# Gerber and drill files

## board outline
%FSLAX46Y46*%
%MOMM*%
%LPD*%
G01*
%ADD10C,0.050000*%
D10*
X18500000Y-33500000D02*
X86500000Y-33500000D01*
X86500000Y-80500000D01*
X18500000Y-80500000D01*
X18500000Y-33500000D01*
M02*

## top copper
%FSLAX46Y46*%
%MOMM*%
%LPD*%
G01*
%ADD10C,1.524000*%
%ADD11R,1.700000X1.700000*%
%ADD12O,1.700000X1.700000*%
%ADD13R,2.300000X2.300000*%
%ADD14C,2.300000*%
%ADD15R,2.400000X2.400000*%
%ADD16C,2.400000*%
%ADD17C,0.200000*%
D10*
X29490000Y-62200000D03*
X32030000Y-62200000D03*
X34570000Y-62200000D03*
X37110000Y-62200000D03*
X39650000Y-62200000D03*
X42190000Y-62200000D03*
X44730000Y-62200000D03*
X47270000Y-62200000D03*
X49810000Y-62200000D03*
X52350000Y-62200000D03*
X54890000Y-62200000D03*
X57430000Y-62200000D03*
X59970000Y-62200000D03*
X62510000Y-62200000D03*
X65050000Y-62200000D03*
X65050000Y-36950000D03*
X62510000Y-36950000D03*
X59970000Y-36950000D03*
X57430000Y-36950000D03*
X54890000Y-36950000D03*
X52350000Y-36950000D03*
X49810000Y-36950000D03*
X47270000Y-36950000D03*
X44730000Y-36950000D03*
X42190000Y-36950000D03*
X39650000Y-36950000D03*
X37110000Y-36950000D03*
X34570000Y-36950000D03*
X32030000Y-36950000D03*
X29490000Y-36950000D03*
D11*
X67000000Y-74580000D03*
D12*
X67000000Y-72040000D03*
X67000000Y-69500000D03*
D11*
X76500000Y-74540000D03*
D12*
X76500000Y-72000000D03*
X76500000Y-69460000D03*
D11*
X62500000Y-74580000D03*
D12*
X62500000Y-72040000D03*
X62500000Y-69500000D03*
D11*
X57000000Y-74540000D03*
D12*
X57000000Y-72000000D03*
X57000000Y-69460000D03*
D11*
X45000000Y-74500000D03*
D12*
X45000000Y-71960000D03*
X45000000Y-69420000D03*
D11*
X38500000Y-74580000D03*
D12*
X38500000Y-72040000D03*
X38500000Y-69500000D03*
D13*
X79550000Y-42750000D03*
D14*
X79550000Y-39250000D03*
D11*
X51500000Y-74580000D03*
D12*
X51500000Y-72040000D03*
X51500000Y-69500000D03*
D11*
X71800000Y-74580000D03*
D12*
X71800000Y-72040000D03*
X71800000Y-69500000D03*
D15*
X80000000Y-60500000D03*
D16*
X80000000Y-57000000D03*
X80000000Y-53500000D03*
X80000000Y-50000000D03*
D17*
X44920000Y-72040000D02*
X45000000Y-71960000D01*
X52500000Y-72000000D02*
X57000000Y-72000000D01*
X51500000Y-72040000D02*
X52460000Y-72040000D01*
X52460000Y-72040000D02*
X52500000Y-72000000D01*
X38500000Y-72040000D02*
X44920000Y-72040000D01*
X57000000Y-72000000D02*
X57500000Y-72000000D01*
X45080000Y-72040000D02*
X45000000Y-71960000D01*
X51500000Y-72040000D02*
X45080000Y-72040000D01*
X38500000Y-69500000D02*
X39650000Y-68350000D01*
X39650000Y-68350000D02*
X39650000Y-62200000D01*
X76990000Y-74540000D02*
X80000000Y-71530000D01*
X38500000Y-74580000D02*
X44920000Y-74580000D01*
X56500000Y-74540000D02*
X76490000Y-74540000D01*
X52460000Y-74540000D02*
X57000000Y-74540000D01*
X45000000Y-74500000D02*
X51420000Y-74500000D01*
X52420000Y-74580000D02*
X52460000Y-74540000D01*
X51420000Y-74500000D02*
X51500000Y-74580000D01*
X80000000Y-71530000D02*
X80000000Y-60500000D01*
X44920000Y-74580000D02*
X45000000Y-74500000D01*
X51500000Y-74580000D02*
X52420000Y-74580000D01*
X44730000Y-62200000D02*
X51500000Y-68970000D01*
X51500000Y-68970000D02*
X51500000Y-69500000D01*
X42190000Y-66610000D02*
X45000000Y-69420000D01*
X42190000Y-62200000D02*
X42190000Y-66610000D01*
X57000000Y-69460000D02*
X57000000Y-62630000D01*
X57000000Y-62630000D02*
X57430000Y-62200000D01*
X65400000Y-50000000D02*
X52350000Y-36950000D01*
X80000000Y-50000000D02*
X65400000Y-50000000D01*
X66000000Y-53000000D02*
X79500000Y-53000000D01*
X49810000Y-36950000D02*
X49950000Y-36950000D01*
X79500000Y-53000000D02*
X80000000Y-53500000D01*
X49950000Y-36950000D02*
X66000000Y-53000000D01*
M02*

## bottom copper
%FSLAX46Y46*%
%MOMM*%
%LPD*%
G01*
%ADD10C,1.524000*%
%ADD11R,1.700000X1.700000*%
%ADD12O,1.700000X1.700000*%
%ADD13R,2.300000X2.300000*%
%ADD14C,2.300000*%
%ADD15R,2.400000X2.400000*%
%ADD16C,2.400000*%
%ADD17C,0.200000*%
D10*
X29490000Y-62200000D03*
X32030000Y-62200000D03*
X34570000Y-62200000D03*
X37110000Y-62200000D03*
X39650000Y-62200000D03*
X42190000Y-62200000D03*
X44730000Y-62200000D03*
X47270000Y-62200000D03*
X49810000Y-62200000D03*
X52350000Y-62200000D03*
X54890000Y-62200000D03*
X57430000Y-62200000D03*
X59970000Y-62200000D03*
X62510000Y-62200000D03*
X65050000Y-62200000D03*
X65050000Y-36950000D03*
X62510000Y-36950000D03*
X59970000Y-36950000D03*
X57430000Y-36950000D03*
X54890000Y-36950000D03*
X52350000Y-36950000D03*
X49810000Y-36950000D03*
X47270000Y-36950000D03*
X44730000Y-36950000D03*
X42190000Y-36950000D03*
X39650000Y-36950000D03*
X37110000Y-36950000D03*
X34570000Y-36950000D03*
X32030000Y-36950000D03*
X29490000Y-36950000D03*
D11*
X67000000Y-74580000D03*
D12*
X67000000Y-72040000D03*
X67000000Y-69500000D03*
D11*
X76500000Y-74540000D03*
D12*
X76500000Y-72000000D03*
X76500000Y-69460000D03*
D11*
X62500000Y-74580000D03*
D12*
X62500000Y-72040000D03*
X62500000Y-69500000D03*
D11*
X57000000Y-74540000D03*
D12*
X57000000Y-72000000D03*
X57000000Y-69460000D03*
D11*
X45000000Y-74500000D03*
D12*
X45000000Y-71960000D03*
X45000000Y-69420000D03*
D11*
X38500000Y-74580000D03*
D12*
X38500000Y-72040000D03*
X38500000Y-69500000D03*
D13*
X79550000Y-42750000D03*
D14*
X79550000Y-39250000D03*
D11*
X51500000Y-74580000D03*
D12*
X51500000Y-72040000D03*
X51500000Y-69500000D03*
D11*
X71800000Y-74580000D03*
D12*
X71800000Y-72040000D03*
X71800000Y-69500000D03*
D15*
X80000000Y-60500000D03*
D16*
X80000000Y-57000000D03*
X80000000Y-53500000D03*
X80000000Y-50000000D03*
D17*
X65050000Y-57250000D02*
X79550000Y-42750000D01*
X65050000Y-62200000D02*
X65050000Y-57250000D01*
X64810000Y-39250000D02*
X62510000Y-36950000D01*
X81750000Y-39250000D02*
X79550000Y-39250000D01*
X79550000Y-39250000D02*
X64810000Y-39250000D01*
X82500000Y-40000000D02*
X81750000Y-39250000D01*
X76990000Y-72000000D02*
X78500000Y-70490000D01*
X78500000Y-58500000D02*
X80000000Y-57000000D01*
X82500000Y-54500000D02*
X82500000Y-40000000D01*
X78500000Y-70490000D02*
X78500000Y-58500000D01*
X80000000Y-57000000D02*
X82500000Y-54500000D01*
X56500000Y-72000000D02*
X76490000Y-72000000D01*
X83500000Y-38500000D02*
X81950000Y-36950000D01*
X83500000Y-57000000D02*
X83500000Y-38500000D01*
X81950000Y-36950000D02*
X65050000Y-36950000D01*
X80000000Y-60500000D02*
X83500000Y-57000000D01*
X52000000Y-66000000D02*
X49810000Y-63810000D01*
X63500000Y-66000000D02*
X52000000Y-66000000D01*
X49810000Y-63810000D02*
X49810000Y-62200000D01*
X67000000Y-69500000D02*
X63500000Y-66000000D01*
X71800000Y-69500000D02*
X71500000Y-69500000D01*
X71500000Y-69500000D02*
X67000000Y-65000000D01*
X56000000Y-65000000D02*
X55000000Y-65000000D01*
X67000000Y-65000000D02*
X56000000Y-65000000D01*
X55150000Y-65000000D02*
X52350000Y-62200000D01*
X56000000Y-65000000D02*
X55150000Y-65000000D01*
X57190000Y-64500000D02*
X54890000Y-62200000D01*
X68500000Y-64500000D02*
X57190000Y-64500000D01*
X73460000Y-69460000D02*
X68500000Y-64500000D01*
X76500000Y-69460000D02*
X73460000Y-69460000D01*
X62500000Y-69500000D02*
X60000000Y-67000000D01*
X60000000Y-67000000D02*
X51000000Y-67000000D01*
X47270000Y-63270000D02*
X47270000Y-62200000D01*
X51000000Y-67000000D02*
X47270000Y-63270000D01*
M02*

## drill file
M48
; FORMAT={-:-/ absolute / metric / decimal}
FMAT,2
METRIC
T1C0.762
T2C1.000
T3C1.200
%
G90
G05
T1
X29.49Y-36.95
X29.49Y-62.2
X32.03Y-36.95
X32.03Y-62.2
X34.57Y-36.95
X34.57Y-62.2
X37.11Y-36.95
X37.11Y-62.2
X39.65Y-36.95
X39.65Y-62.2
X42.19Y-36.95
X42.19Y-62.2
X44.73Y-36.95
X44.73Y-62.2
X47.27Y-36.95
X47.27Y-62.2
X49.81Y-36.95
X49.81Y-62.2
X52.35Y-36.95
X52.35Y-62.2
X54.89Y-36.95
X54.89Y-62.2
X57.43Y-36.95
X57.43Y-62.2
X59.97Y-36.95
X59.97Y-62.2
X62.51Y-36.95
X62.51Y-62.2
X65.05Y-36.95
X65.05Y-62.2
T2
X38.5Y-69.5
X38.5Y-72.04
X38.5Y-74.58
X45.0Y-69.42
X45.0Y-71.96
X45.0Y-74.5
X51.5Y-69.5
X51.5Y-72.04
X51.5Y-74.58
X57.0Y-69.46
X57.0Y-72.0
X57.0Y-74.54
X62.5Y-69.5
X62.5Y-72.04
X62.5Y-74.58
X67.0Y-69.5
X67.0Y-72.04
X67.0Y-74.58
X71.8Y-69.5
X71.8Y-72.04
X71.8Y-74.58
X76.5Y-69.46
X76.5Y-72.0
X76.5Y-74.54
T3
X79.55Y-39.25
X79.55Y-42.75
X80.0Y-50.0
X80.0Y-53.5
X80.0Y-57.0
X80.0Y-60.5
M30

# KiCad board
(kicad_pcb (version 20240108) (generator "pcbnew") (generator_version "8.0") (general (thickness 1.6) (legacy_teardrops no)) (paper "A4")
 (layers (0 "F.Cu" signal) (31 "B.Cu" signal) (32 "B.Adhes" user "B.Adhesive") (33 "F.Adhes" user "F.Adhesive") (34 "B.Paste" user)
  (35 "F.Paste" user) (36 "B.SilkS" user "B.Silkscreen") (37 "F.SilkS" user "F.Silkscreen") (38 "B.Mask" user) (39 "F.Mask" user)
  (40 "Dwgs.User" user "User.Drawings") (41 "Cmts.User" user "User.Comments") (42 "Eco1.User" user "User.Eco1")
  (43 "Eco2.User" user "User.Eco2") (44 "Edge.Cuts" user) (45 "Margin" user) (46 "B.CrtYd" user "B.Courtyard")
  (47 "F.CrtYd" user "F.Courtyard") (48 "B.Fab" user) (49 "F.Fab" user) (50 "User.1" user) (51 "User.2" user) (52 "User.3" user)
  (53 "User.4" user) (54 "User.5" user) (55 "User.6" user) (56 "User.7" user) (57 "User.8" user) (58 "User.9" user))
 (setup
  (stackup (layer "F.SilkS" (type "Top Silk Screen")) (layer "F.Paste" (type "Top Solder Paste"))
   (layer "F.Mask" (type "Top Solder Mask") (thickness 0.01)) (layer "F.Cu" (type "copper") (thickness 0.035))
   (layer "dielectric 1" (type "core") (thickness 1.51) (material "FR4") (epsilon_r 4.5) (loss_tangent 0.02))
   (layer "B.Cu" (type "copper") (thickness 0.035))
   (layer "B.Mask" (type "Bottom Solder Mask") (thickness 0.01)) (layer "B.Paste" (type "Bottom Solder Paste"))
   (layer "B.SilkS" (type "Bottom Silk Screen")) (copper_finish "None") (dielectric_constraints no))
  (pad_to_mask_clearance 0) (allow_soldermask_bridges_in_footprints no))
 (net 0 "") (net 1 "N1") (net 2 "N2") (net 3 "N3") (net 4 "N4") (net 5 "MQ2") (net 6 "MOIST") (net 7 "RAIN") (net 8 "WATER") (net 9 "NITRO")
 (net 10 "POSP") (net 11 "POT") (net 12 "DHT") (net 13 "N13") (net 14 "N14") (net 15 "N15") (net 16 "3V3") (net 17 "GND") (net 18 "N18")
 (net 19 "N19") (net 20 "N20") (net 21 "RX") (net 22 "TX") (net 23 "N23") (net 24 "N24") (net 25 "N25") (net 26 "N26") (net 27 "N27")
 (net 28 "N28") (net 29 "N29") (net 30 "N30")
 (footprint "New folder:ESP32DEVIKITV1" (layer "F.Cu") (at 29.49 62.2)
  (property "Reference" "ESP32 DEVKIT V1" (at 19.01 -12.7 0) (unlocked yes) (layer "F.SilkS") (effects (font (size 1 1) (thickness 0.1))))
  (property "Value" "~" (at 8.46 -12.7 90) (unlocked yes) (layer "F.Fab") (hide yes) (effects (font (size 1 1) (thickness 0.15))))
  (pad "1" thru_hole circle (at 0 0) (size 1.524 1.524) (drill 0.762) (layers "*.Cu" "*.Mask") (remove_unused_layers no) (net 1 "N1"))
  (pad "2" thru_hole circle (at 2.54 0) (size 1.524 1.524) (drill 0.762) (layers "*.Cu" "*.Mask") (remove_unused_layers no) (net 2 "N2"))
  (pad "3" thru_hole circle (at 5.08 0) (size 1.524 1.524) (drill 0.762) (layers "*.Cu" "*.Mask") (remove_unused_layers no) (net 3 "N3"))
  (pad "4" thru_hole circle (at 7.62 0) (size 1.524 1.524) (drill 0.762) (layers "*.Cu" "*.Mask") (remove_unused_layers no) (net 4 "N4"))
  (pad "5" thru_hole circle (at 10.16 0) (size 1.524 1.524) (drill 0.762) (layers "*.Cu" "*.Mask") (remove_unused_layers no) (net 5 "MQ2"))
  (pad "6" thru_hole circle (at 12.7 0) (size 1.524 1.524) (drill 0.762) (layers "*.Cu" "*.Mask") (remove_unused_layers no) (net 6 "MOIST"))
  (pad "7" thru_hole circle (at 15.24 0) (size 1.524 1.524) (drill 0.762) (layers "*.Cu" "*.Mask") (remove_unused_layers no) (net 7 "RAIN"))
  (pad "8" thru_hole circle (at 17.78 0) (size 1.524 1.524) (drill 0.762) (layers "*.Cu" "*.Mask") (remove_unused_layers no) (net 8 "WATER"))
  (pad "9" thru_hole circle (at 20.32 0) (size 1.524 1.524) (drill 0.762) (layers "*.Cu" "*.Mask") (remove_unused_layers no) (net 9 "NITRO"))
  (pad "10" thru_hole circle (at 22.86 0) (size 1.524 1.524) (drill 0.762) (layers "*.Cu" "*.Mask") (remove_unused_layers no)
   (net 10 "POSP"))
  (pad "11" thru_hole circle (at 25.4 0) (size 1.524 1.524) (drill 0.762) (layers "*.Cu" "*.Mask") (remove_unused_layers no) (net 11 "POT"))
  (pad "12" thru_hole circle (at 27.94 0) (size 1.524 1.524) (drill 0.762) (layers "*.Cu" "*.Mask") (remove_unused_layers no) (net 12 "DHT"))
  (pad "13" thru_hole circle (at 30.48 0) (size 1.524 1.524) (drill 0.762) (layers "*.Cu" "*.Mask") (remove_unused_layers no) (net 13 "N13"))
  (pad "14" thru_hole circle (at 33.02 0) (size 1.524 1.524) (drill 0.762) (layers "*.Cu" "*.Mask") (remove_unused_layers no) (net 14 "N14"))
  (pad "15" thru_hole circle (at 35.56 0) (size 1.524 1.524) (drill 0.762) (layers "*.Cu" "*.Mask") (remove_unused_layers no) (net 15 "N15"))
  (pad "16" thru_hole circle (at 35.56 -25.25) (size 1.524 1.524) (drill 0.762) (layers "*.Cu" "*.Mask") (remove_unused_layers no)
   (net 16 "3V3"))
  (pad "17" thru_hole circle (at 33.02 -25.25) (size 1.524 1.524) (drill 0.762) (layers "*.Cu" "*.Mask") (remove_unused_layers no)
   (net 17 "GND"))
  (pad "18" thru_hole circle (at 30.48 -25.25) (size 1.524 1.524) (drill 0.762) (layers "*.Cu" "*.Mask") (remove_unused_layers no)
   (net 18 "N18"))
  (pad "19" thru_hole circle (at 27.94 -25.25) (size 1.524 1.524) (drill 0.762) (layers "*.Cu" "*.Mask") (remove_unused_layers no)
   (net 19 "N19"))
  (pad "20" thru_hole circle (at 25.4 -25.25) (size 1.524 1.524) (drill 0.762) (layers "*.Cu" "*.Mask") (remove_unused_layers no)
   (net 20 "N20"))
  (pad "21" thru_hole circle (at 22.86 -25.25) (size 1.524 1.524) (drill 0.762) (layers "*.Cu" "*.Mask") (remove_unused_layers no)
   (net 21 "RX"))
  (pad "22" thru_hole circle (at 20.32 -25.25) (size 1.524 1.524) (drill 0.762) (layers "*.Cu" "*.Mask") (remove_unused_layers no)
   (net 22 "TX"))
  (pad "23" thru_hole circle (at 17.78 -25.25) (size 1.524 1.524) (drill 0.762) (layers "*.Cu" "*.Mask") (remove_unused_layers no)
   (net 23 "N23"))
  (pad "24" thru_hole circle (at 15.24 -25.25) (size 1.524 1.524) (drill 0.762) (layers "*.Cu" "*.Mask") (remove_unused_layers no)
   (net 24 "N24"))
  (pad "25" thru_hole circle (at 12.7 -25.25) (size 1.524 1.524) (drill 0.762) (layers "*.Cu" "*.Mask") (remove_unused_layers no)
   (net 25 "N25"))
  (pad "26" thru_hole circle (at 10.16 -25.25) (size 1.524 1.524) (drill 0.762) (layers "*.Cu" "*.Mask") (remove_unused_layers no)
   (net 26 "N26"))
  (pad "27" thru_hole circle (at 7.62 -25.25) (size 1.524 1.524) (drill 0.762) (layers "*.Cu" "*.Mask") (remove_unused_layers no)
   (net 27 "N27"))
  (pad "28" thru_hole circle (at 5.08 -25.25) (size 1.524 1.524) (drill 0.762) (layers "*.Cu" "*.Mask") (remove_unused_layers no)
   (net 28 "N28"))
  (pad "29" thru_hole circle (at 2.54 -25.25) (size 1.524 1.524) (drill 0.762) (layers "*.Cu" "*.Mask") (remove_unused_layers no)
   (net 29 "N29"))
  (pad "30" thru_hole circle (at 0 -25.25) (size 1.524 1.524) (drill 0.762) (layers "*.Cu" "*.Mask") (remove_unused_layers no)
   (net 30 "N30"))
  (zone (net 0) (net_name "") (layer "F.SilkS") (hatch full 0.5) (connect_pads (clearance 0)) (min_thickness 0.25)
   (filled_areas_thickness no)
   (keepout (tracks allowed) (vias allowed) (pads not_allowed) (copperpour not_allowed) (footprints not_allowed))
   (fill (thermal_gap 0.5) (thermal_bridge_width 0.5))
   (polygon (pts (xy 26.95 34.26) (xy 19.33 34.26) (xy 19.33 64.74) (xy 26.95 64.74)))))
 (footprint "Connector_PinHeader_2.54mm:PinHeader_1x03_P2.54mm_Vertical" (layer "F.Cu") (at 67 74.58 180)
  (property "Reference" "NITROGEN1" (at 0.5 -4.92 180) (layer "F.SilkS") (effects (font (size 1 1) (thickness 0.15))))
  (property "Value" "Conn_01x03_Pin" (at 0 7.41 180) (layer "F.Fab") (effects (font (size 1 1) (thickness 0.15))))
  (pad "1" thru_hole rect (at 0 0 180) (size 1.7 1.7) (drill 1) (layers "*.Cu" "*.Mask") (remove_unused_layers no) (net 16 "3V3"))
  (pad "2" thru_hole oval (at 0 2.54 180) (size 1.7 1.7) (drill 1) (layers "*.Cu" "*.Mask") (remove_unused_layers no) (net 17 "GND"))
  (pad "3" thru_hole oval (at 0 5.08 180) (size 1.7 1.7) (drill 1) (layers "*.Cu" "*.Mask") (remove_unused_layers no) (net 9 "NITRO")))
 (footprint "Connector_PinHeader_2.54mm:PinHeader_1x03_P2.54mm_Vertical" (layer "F.Cu") (at 76.5 74.54 180)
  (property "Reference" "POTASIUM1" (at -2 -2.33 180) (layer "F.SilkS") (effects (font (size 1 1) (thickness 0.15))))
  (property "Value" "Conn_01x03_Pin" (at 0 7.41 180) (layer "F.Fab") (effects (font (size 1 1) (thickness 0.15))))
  (pad "1" thru_hole rect (at 0 0 180) (size 1.7 1.7) (drill 1) (layers "*.Cu" "*.Mask") (remove_unused_layers no) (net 16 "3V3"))
  (pad "2" thru_hole oval (at 0 2.54 180) (size 1.7 1.7) (drill 1) (layers "*.Cu" "*.Mask") (remove_unused_layers no) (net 17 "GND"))
  (pad "3" thru_hole oval (at 0 5.08 180) (size 1.7 1.7) (drill 1) (layers "*.Cu" "*.Mask") (remove_unused_layers no) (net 11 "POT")))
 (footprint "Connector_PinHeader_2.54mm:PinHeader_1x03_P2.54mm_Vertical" (layer "F.Cu") (at 62.5 74.58 180)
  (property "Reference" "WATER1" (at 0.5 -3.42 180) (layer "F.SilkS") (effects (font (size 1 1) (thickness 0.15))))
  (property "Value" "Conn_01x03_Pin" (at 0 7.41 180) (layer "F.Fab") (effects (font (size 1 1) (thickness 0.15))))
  (pad "1" thru_hole rect (at 0 0 180) (size 1.7 1.7) (drill 1) (layers "*.Cu" "*.Mask") (remove_unused_layers no) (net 16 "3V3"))
  (pad "2" thru_hole oval (at 0 2.54 180) (size 1.7 1.7) (drill 1) (layers "*.Cu" "*.Mask") (remove_unused_layers no) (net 17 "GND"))
  (pad "3" thru_hole oval (at 0 5.08 180) (size 1.7 1.7) (drill 1) (layers "*.Cu" "*.Mask") (remove_unused_layers no) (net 8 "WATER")))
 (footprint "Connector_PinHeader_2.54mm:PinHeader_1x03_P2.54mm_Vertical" (layer "F.Cu") (at 57 74.54 180)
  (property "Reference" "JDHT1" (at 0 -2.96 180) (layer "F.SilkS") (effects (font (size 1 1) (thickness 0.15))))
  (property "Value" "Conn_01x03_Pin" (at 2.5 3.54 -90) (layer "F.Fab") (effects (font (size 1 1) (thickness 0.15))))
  (pad "1" thru_hole rect (at 0 0 180) (size 1.7 1.7) (drill 1) (layers "*.Cu" "*.Mask") (remove_unused_layers no) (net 16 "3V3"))
  (pad "2" thru_hole oval (at 0 2.54 180) (size 1.7 1.7) (drill 1) (layers "*.Cu" "*.Mask") (remove_unused_layers no) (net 17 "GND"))
  (pad "3" thru_hole oval (at 0 5.08 180) (size 1.7 1.7) (drill 1) (layers "*.Cu" "*.Mask") (remove_unused_layers no) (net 12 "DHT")))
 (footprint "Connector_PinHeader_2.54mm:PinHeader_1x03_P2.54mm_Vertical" (layer "F.Cu") (at 45 74.5 180)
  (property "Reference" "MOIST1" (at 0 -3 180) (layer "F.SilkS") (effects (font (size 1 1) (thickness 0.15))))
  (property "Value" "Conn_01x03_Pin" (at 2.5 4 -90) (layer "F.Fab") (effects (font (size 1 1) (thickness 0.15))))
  (pad "1" thru_hole rect (at 0 0 180) (size 1.7 1.7) (drill 1) (layers "*.Cu" "*.Mask") (remove_unused_layers no) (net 16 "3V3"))
  (pad "2" thru_hole oval (at 0 2.54 180) (size 1.7 1.7) (drill 1) (layers "*.Cu" "*.Mask") (remove_unused_layers no) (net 17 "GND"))
  (pad "3" thru_hole oval (at 0 5.08 180) (size 1.7 1.7) (drill 1) (layers "*.Cu" "*.Mask") (remove_unused_layers no) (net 6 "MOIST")))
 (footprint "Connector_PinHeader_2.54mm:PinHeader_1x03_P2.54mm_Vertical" (layer "F.Cu") (at 38.5 74.58 180)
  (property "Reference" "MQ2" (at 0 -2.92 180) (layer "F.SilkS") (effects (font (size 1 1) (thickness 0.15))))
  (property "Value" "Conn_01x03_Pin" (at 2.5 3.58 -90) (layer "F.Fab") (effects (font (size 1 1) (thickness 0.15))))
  (pad "1" thru_hole rect (at 0 0 180) (size 1.7 1.7) (drill 1) (layers "*.Cu" "*.Mask") (remove_unused_layers no) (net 16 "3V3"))
  (pad "2" thru_hole oval (at 0 2.54 180) (size 1.7 1.7) (drill 1) (layers "*.Cu" "*.Mask") (remove_unused_layers no) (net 17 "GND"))
  (pad "3" thru_hole oval (at 0 5.08 180) (size 1.7 1.7) (drill 1) (layers "*.Cu" "*.Mask") (remove_unused_layers no) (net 5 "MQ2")))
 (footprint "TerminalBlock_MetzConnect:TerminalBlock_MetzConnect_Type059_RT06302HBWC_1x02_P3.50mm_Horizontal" (layer "F.Cu")
  (at 79.55 42.75 90)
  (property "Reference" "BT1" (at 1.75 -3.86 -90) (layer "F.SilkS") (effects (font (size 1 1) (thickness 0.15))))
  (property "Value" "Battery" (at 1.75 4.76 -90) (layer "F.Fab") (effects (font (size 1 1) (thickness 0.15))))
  (pad "1" thru_hole rect (at 0 0 90) (size 2.3 2.3) (drill 1.2) (layers "*.Cu" "*.Mask") (remove_unused_layers no) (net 15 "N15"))
  (pad "2" thru_hole circle (at 3.5 0 90) (size 2.3 2.3) (drill 1.2) (layers "*.Cu" "*.Mask") (remove_unused_layers no) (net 17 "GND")))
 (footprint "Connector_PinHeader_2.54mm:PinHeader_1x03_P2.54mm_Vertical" (layer "F.Cu") (at 51.5 74.58 180)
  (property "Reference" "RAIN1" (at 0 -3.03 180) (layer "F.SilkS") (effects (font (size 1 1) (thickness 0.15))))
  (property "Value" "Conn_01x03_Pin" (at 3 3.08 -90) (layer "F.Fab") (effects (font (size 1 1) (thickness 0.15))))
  (pad "1" thru_hole rect (at 0 0 180) (size 1.7 1.7) (drill 1) (layers "*.Cu" "*.Mask") (remove_unused_layers no) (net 16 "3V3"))
  (pad "2" thru_hole oval (at 0 2.54 180) (size 1.7 1.7) (drill 1) (layers "*.Cu" "*.Mask") (remove_unused_layers no) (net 17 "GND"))
  (pad "3" thru_hole oval (at 0 5.08 180) (size 1.7 1.7) (drill 1) (layers "*.Cu" "*.Mask") (remove_unused_layers no) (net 7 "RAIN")))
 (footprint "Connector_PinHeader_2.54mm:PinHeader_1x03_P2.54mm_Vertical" (layer "F.Cu") (at 71.8 74.58 180)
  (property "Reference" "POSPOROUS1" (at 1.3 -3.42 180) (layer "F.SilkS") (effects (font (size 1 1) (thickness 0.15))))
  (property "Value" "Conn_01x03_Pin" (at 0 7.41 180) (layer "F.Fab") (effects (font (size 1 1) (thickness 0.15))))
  (pad "1" thru_hole rect (at 0 0 180) (size 1.7 1.7) (drill 1) (layers "*.Cu" "*.Mask") (remove_unused_layers no) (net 16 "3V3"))
  (pad "2" thru_hole oval (at 0 2.54 180) (size 1.7 1.7) (drill 1) (layers "*.Cu" "*.Mask") (remove_unused_layers no) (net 17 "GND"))
  (pad "3" thru_hole oval (at 0 5.08 180) (size 1.7 1.7) (drill 1) (layers "*.Cu" "*.Mask") (remove_unused_layers no) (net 10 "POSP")))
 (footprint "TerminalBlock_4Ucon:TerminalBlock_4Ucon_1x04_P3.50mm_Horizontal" (layer "F.Cu") (at 80 60.5 90)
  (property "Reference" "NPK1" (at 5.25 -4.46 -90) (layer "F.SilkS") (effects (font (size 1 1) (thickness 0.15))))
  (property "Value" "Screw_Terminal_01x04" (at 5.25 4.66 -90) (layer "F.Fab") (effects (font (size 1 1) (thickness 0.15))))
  (pad "1" thru_hole rect (at 0 0 90) (size 2.4 2.4) (drill 1.2) (layers "*.Cu" "*.Mask") (remove_unused_layers no) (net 16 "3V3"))
  (pad "2" thru_hole circle (at 3.5 0 90) (size 2.4 2.4) (drill 1.2) (layers "*.Cu" "*.Mask") (remove_unused_layers no) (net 17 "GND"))
  (pad "3" thru_hole circle (at 7 0 90) (size 2.4 2.4) (drill 1.2) (layers "*.Cu" "*.Mask") (remove_unused_layers no) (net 22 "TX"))
  (pad "4" thru_hole circle (at 10.5 0 90) (size 2.4 2.4) (drill 1.2) (layers "*.Cu" "*.Mask") (remove_unused_layers no) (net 21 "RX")))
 (gr_rect (start 18.5 33.5) (end 86.5 80.5) (stroke (width 0.05) (type default)) (fill none) (layer "Edge.Cuts"))
 (segment (start 65.05 57.25) (end 79.55 42.75) (width 0.2) (layer "B.Cu") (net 15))
 (segment (start 65.05 62.2) (end 65.05 57.25) (width 0.2) (layer "B.Cu") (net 15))
 (segment (start 44.92 72.04) (end 45 71.96) (width 0.2) (layer "F.Cu") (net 17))
 (segment (start 52.5 72) (end 57 72) (width 0.2) (layer "F.Cu") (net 17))
 (segment (start 51.5 72.04) (end 52.46 72.04) (width 0.2) (layer "F.Cu") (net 17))
 (segment (start 52.46 72.04) (end 52.5 72) (width 0.2) (layer "F.Cu") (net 17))
 (segment (start 38.5 72.04) (end 44.92 72.04) (width 0.2) (layer "F.Cu") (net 17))
 (segment (start 57 72) (end 57.5 72) (width 0.2) (layer "F.Cu") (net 17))
 (segment (start 45.08 72.04) (end 45 71.96) (width 0.2) (layer "F.Cu") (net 17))
 (segment (start 51.5 72.04) (end 45.08 72.04) (width 0.2) (layer "F.Cu") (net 17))
 (segment (start 64.81 39.25) (end 62.51 36.95) (width 0.2) (layer "B.Cu") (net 17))
 (segment (start 81.75 39.25) (end 79.55 39.25) (width 0.2) (layer "B.Cu") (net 17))
 (segment (start 79.55 39.25) (end 64.81 39.25) (width 0.2) (layer "B.Cu") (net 17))
 (segment (start 82.5 40) (end 81.75 39.25) (width 0.2) (layer "B.Cu") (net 17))
 (segment (start 76.99 72) (end 78.5 70.49) (width 0.2) (layer "B.Cu") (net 17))
 (segment (start 78.5 58.5) (end 80 57) (width 0.2) (layer "B.Cu") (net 17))
 (segment (start 82.5 54.5) (end 82.5 40) (width 0.2) (layer "B.Cu") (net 17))
 (segment (start 78.5 70.49) (end 78.5 58.5) (width 0.2) (layer "B.Cu") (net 17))
 (segment (start 80 57) (end 82.5 54.5) (width 0.2) (layer "B.Cu") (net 17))
 (segment (start 56.5 72) (end 76.49 72) (width 0.2) (layer "B.Cu") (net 17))
 (segment (start 38.5 69.5) (end 39.65 68.35) (width 0.2) (layer "F.Cu") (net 5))
 (segment (start 39.65 68.35) (end 39.65 62.2) (width 0.2) (layer "F.Cu") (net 5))
 (segment (start 76.99 74.54) (end 80 71.53) (width 0.2) (layer "F.Cu") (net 16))
 (segment (start 38.5 74.58) (end 44.92 74.58) (width 0.2) (layer "F.Cu") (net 16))
 (segment (start 56.5 74.54) (end 76.49 74.54) (width 0.2) (layer "F.Cu") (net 16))
 (segment (start 52.46 74.54) (end 57 74.54) (width 0.2) (layer "F.Cu") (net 16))
 (segment (start 45 74.5) (end 51.42 74.5) (width 0.2) (layer "F.Cu") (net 16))
 (segment (start 52.42 74.58) (end 52.46 74.54) (width 0.2) (layer "F.Cu") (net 16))
 (segment (start 51.42 74.5) (end 51.5 74.58) (width 0.2) (layer "F.Cu") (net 16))
 (segment (start 80 71.53) (end 80 60.5) (width 0.2) (layer "F.Cu") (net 16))
 (segment (start 44.92 74.58) (end 45 74.5) (width 0.2) (layer "F.Cu") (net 16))
 (segment (start 51.5 74.58) (end 52.42 74.58) (width 0.2) (layer "F.Cu") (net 16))
 (segment (start 83.5 38.5) (end 81.95 36.95) (width 0.2) (layer "B.Cu") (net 16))
 (segment (start 83.5 57) (end 83.5 38.5) (width 0.2) (layer "B.Cu") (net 16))
 (segment (start 81.95 36.95) (end 65.05 36.95) (width 0.2) (layer "B.Cu") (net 16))
 (segment (start 80 60.5) (end 83.5 57) (width 0.2) (layer "B.Cu") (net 16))
 (segment (start 44.73 62.2) (end 51.5 68.97) (width 0.2) (layer "F.Cu") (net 7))
 (segment (start 51.5 68.97) (end 51.5 69.5) (width 0.2) (layer "F.Cu") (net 7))
 (segment (start 42.19 66.61) (end 45 69.42) (width 0.2) (layer "F.Cu") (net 6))
 (segment (start 42.19 62.2) (end 42.19 66.61) (width 0.2) (layer "F.Cu") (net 6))
 (segment (start 57 69.46) (end 57 62.63) (width 0.2) (layer "F.Cu") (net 12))
 (segment (start 57 62.63) (end 57.43 62.2) (width 0.2) (layer "F.Cu") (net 12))
 (segment (start 65.4 50) (end 52.35 36.95) (width 0.2) (layer "F.Cu") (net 21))
 (segment (start 80 50) (end 65.4 50) (width 0.2) (layer "F.Cu") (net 21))
 (segment (start 66 53) (end 79.5 53) (width 0.2) (layer "F.Cu") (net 22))
 (segment (start 49.81 36.95) (end 49.95 36.95) (width 0.2) (layer "F.Cu") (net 22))
 (segment (start 79.5 53) (end 80 53.5) (width 0.2) (layer "F.Cu") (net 22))
 (segment (start 49.95 36.95) (end 66 53) (width 0.2) (layer "F.Cu") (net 22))
 (segment (start 52 66) (end 49.81 63.81) (width 0.2) (layer "B.Cu") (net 9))
 (segment (start 63.5 66) (end 52 66) (width 0.2) (layer "B.Cu") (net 9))
 (segment (start 49.81 63.81) (end 49.81 62.2) (width 0.2) (layer "B.Cu") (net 9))
 (segment (start 67 69.5) (end 63.5 66) (width 0.2) (layer "B.Cu") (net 9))
 (segment (start 71.8 69.5) (end 71.5 69.5) (width 0.2) (layer "B.Cu") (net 10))
 (segment (start 71.5 69.5) (end 67 65) (width 0.2) (layer "B.Cu") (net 10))
 (segment (start 56 65) (end 55 65) (width 0.2) (layer "B.Cu") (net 10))
 (segment (start 67 65) (end 56 65) (width 0.2) (layer "B.Cu") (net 10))
 (segment (start 55.15 65) (end 52.35 62.2) (width 0.2) (layer "B.Cu") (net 10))
 (segment (start 56 65) (end 55.15 65) (width 0.2) (layer "B.Cu") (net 10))
 (segment (start 57.19 64.5) (end 54.89 62.2) (width 0.2) (layer "B.Cu") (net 11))
 (segment (start 68.5 64.5) (end 57.19 64.5) (width 0.2) (layer "B.Cu") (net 11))
 (segment (start 73.46 69.46) (end 68.5 64.5) (width 0.2) (layer "B.Cu") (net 11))
 (segment (start 76.5 69.46) (end 73.46 69.46) (width 0.2) (layer "B.Cu") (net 11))
 (segment (start 62.5 69.5) (end 60 67) (width 0.2) (layer "B.Cu") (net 8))
 (segment (start 60 67) (end 51 67) (width 0.2) (layer "B.Cu") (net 8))
 (segment (start 47.27 63.27) (end 47.27 62.2) (width 0.2) (layer "B.Cu") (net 8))
 (segment (start 51 67) (end 47.27 63.27) (width 0.2) (layer "B.Cu") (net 8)))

